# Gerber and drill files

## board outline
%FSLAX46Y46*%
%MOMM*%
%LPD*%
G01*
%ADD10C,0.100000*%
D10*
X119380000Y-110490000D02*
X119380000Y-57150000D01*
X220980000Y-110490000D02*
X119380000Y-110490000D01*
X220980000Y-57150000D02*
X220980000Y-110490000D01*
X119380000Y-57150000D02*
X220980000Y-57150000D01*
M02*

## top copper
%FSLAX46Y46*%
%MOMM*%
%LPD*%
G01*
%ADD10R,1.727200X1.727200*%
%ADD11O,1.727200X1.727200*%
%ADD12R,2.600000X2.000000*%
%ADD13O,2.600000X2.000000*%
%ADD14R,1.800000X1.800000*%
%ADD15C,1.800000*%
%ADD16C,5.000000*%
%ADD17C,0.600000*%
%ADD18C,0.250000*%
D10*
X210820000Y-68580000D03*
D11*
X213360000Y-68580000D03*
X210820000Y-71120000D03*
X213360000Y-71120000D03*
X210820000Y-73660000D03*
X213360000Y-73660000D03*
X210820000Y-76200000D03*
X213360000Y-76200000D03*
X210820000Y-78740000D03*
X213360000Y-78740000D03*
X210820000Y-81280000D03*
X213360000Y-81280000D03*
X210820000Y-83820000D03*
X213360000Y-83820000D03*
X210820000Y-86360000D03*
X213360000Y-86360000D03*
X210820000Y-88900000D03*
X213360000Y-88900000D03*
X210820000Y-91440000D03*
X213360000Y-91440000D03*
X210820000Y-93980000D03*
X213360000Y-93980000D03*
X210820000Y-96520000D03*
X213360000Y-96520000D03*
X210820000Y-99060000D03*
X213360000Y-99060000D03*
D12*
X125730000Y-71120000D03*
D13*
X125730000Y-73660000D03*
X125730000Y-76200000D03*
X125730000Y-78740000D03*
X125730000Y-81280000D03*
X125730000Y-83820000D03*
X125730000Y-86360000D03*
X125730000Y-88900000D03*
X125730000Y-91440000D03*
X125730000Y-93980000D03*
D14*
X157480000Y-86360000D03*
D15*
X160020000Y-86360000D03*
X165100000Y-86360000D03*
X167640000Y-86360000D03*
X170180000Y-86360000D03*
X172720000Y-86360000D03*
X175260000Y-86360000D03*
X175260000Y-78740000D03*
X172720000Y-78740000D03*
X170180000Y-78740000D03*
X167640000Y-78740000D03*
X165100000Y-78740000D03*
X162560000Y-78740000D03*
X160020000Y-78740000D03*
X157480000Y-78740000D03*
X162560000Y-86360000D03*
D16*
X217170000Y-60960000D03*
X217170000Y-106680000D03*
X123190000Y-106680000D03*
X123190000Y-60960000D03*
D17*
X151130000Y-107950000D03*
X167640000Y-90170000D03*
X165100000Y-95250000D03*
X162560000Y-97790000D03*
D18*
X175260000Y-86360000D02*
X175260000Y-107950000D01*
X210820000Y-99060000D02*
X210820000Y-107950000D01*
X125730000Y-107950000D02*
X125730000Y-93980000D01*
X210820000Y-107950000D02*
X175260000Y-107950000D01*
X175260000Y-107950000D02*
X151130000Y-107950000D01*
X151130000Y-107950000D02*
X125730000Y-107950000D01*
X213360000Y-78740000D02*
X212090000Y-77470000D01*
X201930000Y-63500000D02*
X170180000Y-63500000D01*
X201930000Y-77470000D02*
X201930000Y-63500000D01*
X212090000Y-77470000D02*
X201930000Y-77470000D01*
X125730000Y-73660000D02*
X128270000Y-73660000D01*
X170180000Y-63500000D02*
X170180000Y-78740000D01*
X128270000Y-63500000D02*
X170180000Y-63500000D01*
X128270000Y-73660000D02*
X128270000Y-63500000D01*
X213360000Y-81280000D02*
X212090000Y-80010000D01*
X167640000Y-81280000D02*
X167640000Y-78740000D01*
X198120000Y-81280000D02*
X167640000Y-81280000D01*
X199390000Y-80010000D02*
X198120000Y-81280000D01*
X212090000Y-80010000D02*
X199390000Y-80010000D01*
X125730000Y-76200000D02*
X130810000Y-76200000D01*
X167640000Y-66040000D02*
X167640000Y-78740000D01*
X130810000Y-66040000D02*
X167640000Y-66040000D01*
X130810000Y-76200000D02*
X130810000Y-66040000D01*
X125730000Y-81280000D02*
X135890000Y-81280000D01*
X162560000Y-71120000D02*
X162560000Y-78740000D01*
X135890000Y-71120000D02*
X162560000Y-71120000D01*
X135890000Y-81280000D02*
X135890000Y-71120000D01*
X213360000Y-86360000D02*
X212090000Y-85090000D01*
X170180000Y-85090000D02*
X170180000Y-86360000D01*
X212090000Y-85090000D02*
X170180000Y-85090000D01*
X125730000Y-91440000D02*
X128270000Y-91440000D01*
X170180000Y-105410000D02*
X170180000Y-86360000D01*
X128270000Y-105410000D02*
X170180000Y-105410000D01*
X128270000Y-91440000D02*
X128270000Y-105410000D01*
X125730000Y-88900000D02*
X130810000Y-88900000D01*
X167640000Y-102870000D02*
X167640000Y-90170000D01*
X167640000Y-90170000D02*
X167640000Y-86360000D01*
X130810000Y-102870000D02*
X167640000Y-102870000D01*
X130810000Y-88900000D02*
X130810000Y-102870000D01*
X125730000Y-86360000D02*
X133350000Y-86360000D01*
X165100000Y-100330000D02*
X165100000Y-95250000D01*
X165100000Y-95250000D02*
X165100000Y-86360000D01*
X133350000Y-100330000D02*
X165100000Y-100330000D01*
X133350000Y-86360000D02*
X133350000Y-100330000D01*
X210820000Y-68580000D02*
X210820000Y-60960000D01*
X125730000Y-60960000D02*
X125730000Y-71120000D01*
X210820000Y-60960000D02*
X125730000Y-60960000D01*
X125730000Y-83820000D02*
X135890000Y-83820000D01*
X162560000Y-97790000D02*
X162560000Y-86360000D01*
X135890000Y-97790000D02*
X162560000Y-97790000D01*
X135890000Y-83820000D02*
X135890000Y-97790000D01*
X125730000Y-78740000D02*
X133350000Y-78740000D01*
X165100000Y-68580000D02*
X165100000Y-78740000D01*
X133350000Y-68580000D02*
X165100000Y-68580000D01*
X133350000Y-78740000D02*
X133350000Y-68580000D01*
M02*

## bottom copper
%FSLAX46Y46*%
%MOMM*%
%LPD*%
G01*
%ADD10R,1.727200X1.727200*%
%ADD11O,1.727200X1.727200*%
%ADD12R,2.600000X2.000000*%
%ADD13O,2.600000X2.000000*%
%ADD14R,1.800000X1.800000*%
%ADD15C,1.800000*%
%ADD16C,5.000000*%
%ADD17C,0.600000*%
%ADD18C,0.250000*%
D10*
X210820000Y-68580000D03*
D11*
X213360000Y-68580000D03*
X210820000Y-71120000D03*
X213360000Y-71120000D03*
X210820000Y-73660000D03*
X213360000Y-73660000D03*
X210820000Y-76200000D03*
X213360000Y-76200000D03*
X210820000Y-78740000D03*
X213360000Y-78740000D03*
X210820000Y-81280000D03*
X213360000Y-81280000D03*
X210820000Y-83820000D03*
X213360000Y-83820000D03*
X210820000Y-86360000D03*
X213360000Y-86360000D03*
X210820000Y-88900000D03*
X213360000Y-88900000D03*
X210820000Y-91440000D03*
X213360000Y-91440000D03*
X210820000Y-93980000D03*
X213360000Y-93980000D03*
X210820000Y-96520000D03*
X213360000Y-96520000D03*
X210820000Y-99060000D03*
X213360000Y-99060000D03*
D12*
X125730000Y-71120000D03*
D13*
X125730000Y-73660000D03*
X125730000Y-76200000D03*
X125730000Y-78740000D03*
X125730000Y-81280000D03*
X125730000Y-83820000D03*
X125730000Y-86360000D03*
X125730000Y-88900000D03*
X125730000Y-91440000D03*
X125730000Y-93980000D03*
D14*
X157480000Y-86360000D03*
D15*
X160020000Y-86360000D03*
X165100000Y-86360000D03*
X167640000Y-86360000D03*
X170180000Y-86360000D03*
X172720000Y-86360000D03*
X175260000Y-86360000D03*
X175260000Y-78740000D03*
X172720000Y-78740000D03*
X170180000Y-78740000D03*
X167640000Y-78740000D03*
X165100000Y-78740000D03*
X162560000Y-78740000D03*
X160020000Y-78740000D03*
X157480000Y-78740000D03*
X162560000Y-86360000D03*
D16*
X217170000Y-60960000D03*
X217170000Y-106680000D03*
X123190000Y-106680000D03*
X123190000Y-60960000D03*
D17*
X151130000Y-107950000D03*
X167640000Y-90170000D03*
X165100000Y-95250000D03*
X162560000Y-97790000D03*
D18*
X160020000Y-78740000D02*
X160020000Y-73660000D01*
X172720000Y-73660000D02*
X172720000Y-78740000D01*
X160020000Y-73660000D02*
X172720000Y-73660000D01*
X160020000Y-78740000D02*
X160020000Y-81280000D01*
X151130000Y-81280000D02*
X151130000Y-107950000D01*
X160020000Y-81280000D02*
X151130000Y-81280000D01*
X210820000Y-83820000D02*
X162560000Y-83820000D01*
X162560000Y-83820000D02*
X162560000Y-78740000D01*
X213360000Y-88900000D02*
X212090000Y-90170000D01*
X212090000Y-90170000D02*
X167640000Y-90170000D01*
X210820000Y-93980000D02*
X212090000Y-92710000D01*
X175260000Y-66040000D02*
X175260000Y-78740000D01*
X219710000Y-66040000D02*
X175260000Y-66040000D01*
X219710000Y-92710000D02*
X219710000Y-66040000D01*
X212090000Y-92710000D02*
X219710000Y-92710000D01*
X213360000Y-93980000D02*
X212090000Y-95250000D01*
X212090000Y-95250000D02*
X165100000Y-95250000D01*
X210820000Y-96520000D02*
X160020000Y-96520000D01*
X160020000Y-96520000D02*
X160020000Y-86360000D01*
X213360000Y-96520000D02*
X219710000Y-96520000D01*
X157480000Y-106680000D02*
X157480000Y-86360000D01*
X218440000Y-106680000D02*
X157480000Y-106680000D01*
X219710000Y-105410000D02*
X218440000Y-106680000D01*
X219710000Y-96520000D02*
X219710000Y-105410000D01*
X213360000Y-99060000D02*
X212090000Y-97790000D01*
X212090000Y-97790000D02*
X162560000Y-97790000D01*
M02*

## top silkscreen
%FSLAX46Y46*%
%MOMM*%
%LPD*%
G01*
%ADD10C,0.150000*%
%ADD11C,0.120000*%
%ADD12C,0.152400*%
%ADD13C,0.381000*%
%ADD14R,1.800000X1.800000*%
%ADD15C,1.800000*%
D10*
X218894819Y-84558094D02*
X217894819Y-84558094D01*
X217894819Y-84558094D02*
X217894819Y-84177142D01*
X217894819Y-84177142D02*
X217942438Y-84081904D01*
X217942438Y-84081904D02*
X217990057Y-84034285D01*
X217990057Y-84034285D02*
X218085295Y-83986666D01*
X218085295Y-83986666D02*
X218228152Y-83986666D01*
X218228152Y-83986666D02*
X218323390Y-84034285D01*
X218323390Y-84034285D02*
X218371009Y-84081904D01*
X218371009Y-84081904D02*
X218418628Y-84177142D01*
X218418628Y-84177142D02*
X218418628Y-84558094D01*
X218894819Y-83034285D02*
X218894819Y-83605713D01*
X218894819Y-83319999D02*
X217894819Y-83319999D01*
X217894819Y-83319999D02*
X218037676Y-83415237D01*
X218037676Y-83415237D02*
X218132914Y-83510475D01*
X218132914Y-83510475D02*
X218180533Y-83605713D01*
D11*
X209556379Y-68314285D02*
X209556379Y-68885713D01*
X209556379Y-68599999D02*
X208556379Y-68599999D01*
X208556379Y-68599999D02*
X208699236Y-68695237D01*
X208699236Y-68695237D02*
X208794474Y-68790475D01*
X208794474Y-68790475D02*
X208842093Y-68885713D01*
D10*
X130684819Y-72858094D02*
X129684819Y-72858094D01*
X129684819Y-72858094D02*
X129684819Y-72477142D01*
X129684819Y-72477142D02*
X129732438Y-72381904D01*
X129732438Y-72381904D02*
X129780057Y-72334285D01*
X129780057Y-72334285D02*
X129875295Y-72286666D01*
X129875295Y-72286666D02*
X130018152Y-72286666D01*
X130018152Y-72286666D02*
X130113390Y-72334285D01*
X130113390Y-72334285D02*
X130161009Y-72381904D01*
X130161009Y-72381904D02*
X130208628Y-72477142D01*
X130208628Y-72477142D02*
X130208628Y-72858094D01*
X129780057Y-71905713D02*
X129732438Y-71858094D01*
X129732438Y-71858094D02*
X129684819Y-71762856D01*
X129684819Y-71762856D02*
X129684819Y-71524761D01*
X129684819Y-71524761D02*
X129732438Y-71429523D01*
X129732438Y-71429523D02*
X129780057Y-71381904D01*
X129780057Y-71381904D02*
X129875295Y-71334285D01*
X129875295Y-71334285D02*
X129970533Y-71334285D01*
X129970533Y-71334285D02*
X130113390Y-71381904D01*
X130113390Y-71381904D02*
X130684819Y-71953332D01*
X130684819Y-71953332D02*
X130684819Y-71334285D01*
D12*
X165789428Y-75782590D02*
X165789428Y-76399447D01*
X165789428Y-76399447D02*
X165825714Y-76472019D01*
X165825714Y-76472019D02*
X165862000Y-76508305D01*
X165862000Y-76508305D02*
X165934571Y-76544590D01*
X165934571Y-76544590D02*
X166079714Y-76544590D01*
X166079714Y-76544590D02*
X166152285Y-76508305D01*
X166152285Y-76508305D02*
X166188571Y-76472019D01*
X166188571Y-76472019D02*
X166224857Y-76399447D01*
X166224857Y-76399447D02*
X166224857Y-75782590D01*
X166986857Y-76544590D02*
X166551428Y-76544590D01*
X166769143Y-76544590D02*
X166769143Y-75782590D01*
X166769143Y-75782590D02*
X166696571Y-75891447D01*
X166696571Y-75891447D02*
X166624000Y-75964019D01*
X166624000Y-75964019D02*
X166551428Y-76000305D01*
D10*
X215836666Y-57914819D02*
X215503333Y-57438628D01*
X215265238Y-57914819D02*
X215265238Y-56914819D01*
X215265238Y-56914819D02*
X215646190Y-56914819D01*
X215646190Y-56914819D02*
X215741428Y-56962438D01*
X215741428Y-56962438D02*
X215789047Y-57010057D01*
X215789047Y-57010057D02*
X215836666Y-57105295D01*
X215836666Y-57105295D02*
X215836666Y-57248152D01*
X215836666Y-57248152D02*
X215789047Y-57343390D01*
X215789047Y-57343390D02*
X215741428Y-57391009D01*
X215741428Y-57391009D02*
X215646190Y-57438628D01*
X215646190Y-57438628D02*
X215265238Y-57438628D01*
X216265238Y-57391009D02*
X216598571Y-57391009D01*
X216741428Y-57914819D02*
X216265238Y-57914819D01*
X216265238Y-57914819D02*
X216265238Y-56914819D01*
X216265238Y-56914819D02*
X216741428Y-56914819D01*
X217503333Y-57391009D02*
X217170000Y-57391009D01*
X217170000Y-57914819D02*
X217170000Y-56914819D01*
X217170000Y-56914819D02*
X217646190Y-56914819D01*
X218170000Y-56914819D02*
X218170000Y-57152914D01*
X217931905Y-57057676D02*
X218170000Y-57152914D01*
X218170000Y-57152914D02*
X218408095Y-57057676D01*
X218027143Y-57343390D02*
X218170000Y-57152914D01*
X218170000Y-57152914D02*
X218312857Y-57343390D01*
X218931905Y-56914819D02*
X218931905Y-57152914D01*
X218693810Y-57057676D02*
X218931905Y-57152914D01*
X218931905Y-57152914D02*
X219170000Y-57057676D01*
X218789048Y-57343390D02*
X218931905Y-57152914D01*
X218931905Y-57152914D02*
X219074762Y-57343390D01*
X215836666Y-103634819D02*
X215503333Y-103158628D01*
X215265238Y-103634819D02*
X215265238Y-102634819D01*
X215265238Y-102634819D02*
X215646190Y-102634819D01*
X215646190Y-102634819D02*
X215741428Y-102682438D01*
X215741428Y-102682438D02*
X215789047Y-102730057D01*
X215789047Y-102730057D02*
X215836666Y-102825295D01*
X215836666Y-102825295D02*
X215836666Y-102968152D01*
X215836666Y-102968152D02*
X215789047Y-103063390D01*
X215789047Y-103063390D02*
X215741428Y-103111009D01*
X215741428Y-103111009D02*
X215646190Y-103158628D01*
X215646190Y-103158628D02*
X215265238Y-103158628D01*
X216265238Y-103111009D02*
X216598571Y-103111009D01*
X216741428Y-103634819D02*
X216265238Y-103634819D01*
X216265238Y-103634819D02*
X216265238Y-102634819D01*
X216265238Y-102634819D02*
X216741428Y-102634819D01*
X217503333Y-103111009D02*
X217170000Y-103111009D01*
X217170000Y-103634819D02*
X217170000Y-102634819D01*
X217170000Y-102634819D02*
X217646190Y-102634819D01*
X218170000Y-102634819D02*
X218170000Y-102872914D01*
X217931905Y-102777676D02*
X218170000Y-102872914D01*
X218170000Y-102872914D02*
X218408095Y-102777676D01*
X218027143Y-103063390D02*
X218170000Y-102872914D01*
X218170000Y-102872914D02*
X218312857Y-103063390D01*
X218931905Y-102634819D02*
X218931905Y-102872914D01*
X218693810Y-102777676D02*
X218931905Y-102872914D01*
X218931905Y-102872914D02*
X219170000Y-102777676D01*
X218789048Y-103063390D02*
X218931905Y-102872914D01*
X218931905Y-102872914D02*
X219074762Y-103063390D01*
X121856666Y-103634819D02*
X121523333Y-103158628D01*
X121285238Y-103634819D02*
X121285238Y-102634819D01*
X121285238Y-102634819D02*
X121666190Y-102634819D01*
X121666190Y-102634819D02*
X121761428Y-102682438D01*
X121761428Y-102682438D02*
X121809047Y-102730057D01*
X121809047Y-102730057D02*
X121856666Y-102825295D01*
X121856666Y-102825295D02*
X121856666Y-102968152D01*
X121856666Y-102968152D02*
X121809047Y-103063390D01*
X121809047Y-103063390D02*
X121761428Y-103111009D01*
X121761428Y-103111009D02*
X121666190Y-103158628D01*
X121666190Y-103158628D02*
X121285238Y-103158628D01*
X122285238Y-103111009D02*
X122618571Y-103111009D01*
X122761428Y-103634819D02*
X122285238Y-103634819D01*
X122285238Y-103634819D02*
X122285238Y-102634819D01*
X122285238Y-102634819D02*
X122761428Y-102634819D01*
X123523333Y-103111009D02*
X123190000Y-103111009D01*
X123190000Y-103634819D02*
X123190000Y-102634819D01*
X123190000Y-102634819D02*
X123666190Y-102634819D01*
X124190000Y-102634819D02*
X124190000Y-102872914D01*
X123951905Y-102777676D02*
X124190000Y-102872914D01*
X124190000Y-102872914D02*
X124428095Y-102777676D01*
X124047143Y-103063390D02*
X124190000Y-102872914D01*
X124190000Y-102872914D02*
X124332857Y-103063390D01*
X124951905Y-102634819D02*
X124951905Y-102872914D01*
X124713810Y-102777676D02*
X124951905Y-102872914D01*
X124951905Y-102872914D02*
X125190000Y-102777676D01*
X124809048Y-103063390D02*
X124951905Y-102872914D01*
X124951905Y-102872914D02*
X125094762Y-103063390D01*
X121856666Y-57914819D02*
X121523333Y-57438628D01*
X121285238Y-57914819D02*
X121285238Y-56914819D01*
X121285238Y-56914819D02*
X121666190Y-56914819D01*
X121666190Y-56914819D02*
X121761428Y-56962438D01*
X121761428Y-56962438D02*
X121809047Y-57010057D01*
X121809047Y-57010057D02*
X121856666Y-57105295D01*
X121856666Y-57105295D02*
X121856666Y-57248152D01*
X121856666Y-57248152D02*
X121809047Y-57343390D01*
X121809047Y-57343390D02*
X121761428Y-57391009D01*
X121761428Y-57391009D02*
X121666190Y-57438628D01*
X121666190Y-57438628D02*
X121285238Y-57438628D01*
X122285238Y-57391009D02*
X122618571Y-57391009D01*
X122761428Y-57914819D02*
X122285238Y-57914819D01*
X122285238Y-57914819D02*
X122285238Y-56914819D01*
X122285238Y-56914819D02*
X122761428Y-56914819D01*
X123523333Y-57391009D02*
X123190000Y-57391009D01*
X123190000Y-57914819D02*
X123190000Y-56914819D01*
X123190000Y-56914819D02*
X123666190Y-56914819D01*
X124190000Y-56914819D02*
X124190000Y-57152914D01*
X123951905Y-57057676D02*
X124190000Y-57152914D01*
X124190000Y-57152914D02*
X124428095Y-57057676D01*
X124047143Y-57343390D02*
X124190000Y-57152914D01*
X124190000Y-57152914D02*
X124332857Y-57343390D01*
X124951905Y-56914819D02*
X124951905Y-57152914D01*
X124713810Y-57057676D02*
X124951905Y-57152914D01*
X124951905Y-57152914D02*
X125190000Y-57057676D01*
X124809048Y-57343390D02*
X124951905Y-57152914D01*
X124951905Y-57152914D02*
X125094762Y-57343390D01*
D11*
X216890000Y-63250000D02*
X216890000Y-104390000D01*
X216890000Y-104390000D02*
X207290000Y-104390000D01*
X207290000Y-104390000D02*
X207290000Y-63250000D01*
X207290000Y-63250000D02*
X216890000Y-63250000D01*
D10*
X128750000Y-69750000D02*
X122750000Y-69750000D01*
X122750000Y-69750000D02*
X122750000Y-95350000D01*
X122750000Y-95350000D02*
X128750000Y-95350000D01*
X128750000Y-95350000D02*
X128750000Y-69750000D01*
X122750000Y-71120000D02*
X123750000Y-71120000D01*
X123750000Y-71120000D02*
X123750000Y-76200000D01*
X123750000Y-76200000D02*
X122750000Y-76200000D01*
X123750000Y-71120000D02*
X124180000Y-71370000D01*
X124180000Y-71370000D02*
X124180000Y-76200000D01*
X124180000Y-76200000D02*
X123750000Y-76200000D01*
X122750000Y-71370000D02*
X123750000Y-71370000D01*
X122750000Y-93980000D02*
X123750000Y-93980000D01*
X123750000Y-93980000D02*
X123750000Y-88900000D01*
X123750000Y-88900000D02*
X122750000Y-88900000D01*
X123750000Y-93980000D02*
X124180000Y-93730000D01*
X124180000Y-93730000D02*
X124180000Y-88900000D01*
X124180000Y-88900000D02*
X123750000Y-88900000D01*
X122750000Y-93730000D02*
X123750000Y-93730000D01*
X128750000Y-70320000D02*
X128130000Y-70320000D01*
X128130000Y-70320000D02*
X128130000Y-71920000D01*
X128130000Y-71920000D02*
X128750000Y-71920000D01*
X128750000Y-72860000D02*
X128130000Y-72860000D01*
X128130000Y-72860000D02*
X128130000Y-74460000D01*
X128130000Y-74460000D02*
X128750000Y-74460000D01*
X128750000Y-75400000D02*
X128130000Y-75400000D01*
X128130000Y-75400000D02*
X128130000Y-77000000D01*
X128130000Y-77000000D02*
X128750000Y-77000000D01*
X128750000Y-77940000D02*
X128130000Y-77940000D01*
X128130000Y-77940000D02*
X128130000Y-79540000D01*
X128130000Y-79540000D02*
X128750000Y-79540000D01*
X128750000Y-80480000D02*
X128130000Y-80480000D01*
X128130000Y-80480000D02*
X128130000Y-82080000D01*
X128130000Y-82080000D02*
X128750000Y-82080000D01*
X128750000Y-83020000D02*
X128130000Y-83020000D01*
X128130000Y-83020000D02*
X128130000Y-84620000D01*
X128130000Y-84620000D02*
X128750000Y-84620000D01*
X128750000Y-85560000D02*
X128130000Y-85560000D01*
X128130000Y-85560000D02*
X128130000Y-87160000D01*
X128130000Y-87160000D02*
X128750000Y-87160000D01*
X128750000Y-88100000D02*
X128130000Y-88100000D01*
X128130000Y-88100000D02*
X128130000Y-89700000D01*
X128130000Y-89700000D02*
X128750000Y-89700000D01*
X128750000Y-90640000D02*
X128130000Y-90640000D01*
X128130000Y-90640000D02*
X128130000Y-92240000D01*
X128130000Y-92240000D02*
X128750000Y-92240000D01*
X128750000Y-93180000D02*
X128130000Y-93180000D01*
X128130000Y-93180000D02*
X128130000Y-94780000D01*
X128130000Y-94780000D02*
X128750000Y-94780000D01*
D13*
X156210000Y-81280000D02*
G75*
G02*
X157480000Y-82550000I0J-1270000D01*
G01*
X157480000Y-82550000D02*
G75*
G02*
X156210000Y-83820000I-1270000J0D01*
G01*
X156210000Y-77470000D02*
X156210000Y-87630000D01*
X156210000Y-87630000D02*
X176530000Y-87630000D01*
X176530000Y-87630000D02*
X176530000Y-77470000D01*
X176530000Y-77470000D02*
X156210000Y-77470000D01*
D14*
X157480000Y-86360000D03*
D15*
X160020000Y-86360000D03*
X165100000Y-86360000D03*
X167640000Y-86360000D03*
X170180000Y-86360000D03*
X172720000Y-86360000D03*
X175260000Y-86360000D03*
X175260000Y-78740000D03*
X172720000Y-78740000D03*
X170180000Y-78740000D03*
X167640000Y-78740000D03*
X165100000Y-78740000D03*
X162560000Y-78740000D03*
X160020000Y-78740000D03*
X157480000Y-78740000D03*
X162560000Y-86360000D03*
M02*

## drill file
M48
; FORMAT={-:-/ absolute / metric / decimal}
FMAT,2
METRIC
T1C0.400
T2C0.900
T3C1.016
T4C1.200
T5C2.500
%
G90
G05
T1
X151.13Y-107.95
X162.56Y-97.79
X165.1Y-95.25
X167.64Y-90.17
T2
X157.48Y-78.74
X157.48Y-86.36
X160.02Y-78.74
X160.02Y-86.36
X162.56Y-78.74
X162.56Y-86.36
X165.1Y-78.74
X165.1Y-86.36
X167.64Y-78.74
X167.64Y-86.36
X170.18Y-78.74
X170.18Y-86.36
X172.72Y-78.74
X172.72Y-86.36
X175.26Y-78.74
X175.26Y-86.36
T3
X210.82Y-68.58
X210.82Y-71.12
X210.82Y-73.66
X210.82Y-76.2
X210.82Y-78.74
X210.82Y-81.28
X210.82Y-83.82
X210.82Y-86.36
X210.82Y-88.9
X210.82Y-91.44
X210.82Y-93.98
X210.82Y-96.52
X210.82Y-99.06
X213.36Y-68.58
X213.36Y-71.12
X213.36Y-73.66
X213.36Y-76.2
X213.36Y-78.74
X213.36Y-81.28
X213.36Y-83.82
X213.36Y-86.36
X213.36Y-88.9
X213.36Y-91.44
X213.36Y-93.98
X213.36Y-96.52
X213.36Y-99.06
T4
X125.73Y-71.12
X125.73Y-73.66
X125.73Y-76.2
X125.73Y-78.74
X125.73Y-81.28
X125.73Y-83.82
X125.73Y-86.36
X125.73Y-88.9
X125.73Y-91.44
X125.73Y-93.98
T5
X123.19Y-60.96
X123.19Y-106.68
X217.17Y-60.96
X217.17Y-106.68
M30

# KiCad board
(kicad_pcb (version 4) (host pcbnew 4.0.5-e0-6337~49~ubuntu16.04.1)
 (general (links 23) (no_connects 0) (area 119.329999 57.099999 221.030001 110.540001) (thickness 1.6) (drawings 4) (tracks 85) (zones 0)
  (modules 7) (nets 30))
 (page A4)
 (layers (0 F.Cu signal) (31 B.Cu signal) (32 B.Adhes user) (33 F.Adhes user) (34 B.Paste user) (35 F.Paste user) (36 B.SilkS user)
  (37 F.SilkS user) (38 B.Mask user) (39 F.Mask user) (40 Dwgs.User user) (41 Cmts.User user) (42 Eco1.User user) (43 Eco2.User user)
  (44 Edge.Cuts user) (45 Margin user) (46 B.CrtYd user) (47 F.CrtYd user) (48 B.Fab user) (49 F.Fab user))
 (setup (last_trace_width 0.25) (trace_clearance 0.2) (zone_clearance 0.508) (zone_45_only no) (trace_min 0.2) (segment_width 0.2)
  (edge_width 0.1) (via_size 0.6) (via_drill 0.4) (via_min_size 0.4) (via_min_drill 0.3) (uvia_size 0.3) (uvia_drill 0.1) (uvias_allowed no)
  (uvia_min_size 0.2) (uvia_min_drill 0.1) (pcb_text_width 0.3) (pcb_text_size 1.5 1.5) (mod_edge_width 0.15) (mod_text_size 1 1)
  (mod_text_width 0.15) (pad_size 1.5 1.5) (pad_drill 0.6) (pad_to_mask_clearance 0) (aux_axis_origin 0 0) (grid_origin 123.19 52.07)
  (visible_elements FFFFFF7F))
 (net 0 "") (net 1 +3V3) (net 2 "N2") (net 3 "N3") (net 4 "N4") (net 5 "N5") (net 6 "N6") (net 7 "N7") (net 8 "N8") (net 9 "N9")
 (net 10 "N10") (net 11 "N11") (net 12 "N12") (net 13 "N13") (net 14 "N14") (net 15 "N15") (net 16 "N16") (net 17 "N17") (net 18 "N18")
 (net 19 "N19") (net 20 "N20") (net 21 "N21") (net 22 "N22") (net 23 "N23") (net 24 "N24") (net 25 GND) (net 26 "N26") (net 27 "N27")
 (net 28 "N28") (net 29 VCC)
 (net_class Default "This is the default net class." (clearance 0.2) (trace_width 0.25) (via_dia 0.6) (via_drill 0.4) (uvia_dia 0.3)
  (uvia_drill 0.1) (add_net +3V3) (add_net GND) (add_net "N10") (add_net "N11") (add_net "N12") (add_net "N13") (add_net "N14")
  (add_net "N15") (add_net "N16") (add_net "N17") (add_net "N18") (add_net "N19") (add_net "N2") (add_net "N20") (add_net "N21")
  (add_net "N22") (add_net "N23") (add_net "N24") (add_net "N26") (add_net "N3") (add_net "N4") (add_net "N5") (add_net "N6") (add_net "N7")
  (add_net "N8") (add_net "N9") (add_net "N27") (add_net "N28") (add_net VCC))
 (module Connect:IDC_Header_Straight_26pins (layer F.Cu) (at 210.82 68.58 270)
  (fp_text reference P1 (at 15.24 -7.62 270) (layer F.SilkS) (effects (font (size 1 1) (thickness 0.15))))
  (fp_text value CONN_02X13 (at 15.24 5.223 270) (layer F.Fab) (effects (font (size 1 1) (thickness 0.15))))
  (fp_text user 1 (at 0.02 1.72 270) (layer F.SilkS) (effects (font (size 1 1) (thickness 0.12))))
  (fp_line (start -5.33 -6.07) (end 35.81 -6.07) (layer F.SilkS) (width 0.12))
  (fp_line (start 35.81 -6.07) (end 35.81 3.53) (layer F.SilkS) (width 0.12))
  (fp_line (start 35.81 3.53) (end -5.33 3.53) (layer F.SilkS) (width 0.12))
  (fp_line (start -5.33 3.53) (end -5.33 -6.07) (layer F.SilkS) (width 0.12))
  (pad 1 thru_hole rect (at 0 0 270) (size 1.7272 1.7272) (drill 1.016) (layers *.Cu *.Mask) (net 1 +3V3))
  (pad 2 thru_hole oval (at 0 -2.54 270) (size 1.7272 1.7272) (drill 1.016) (layers *.Cu *.Mask) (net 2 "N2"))
  (pad 3 thru_hole oval (at 2.54 0 270) (size 1.7272 1.7272) (drill 1.016) (layers *.Cu *.Mask) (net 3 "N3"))
  (pad 4 thru_hole oval (at 2.54 -2.54 270) (size 1.7272 1.7272) (drill 1.016) (layers *.Cu *.Mask) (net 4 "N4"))
  (pad 5 thru_hole oval (at 5.08 0 270) (size 1.7272 1.7272) (drill 1.016) (layers *.Cu *.Mask) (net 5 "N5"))
  (pad 6 thru_hole oval (at 5.08 -2.54 270) (size 1.7272 1.7272) (drill 1.016) (layers *.Cu *.Mask) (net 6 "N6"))
  (pad 7 thru_hole oval (at 7.62 0 270) (size 1.7272 1.7272) (drill 1.016) (layers *.Cu *.Mask) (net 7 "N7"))
  (pad 8 thru_hole oval (at 7.62 -2.54 270) (size 1.7272 1.7272) (drill 1.016) (layers *.Cu *.Mask) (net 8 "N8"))
  (pad 9 thru_hole oval (at 10.16 0 270) (size 1.7272 1.7272) (drill 1.016) (layers *.Cu *.Mask) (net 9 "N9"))
  (pad 10 thru_hole oval (at 10.16 -2.54 270) (size 1.7272 1.7272) (drill 1.016) (layers *.Cu *.Mask) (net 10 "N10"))
  (pad 11 thru_hole oval (at 12.7 0 270) (size 1.7272 1.7272) (drill 1.016) (layers *.Cu *.Mask) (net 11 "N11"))
  (pad 12 thru_hole oval (at 12.7 -2.54 270) (size 1.7272 1.7272) (drill 1.016) (layers *.Cu *.Mask) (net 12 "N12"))
  (pad 13 thru_hole oval (at 15.24 0 270) (size 1.7272 1.7272) (drill 1.016) (layers *.Cu *.Mask) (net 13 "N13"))
  (pad 14 thru_hole oval (at 15.24 -2.54 270) (size 1.7272 1.7272) (drill 1.016) (layers *.Cu *.Mask) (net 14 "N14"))
  (pad 15 thru_hole oval (at 17.78 0 270) (size 1.7272 1.7272) (drill 1.016) (layers *.Cu *.Mask) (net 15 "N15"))
  (pad 16 thru_hole oval (at 17.78 -2.54 270) (size 1.7272 1.7272) (drill 1.016) (layers *.Cu *.Mask) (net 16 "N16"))
  (pad 17 thru_hole oval (at 20.32 0 270) (size 1.7272 1.7272) (drill 1.016) (layers *.Cu *.Mask) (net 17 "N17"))
  (pad 18 thru_hole oval (at 20.32 -2.54 270) (size 1.7272 1.7272) (drill 1.016) (layers *.Cu *.Mask) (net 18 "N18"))
  (pad 19 thru_hole oval (at 22.86 0 270) (size 1.7272 1.7272) (drill 1.016) (layers *.Cu *.Mask) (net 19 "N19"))
  (pad 20 thru_hole oval (at 22.86 -2.54 270) (size 1.7272 1.7272) (drill 1.016) (layers *.Cu *.Mask) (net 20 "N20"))
  (pad 21 thru_hole oval (at 25.4 0 270) (size 1.7272 1.7272) (drill 1.016) (layers *.Cu *.Mask) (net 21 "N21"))
  (pad 22 thru_hole oval (at 25.4 -2.54 270) (size 1.7272 1.7272) (drill 1.016) (layers *.Cu *.Mask) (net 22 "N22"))
  (pad 23 thru_hole oval (at 27.94 0 270) (size 1.7272 1.7272) (drill 1.016) (layers *.Cu *.Mask) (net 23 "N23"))
  (pad 24 thru_hole oval (at 27.94 -2.54 270) (size 1.7272 1.7272) (drill 1.016) (layers *.Cu *.Mask) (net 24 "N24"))
  (pad 25 thru_hole oval (at 30.48 0 270) (size 1.7272 1.7272) (drill 1.016) (layers *.Cu *.Mask) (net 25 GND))
  (pad 26 thru_hole oval (at 30.48 -2.54 270) (size 1.7272 1.7272) (drill 1.016) (layers *.Cu *.Mask) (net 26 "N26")))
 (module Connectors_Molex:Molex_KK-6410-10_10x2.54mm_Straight (layer F.Cu) (at 125.73 71.12 270)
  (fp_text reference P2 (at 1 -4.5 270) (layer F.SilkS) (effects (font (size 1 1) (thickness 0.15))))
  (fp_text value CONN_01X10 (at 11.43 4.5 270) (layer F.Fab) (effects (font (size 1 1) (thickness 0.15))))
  (fp_line (start -1.37 -3.02) (end -1.37 2.98) (layer F.SilkS) (width 0.15))
  (fp_line (start -1.37 2.98) (end 24.23 2.98) (layer F.SilkS) (width 0.15))
  (fp_line (start 24.23 2.98) (end 24.23 -3.02) (layer F.SilkS) (width 0.15))
  (fp_line (start 24.23 -3.02) (end -1.37 -3.02) (layer F.SilkS) (width 0.15))
  (fp_line (start 0 2.98) (end 0 1.98) (layer F.SilkS) (width 0.15))
  (fp_line (start 0 1.98) (end 5.08 1.98) (layer F.SilkS) (width 0.15))
  (fp_line (start 5.08 1.98) (end 5.08 2.98) (layer F.SilkS) (width 0.15))
  (fp_line (start 0 1.98) (end 0.25 1.55) (layer F.SilkS) (width 0.15))
  (fp_line (start 0.25 1.55) (end 5.08 1.55) (layer F.SilkS) (width 0.15))
  (fp_line (start 5.08 1.55) (end 5.08 1.98) (layer F.SilkS) (width 0.15))
  (fp_line (start 0.25 2.98) (end 0.25 1.98) (layer F.SilkS) (width 0.15))
  (fp_line (start 22.86 2.98) (end 22.86 1.98) (layer F.SilkS) (width 0.15))
  (fp_line (start 22.86 1.98) (end 17.78 1.98) (layer F.SilkS) (width 0.15))
  (fp_line (start 17.78 1.98) (end 17.78 2.98) (layer F.SilkS) (width 0.15))
  (fp_line (start 22.86 1.98) (end 22.61 1.55) (layer F.SilkS) (width 0.15))
  (fp_line (start 22.61 1.55) (end 17.78 1.55) (layer F.SilkS) (width 0.15))
  (fp_line (start 17.78 1.55) (end 17.78 1.98) (layer F.SilkS) (width 0.15))
  (fp_line (start 22.61 2.98) (end 22.61 1.98) (layer F.SilkS) (width 0.15))
  (fp_line (start -0.8 -3.02) (end -0.8 -2.4) (layer F.SilkS) (width 0.15))
  (fp_line (start -0.8 -2.4) (end 0.8 -2.4) (layer F.SilkS) (width 0.15))
  (fp_line (start 0.8 -2.4) (end 0.8 -3.02) (layer F.SilkS) (width 0.15))
  (fp_line (start 1.74 -3.02) (end 1.74 -2.4) (layer F.SilkS) (width 0.15))
  (fp_line (start 1.74 -2.4) (end 3.34 -2.4) (layer F.SilkS) (width 0.15))
  (fp_line (start 3.34 -2.4) (end 3.34 -3.02) (layer F.SilkS) (width 0.15))
  (fp_line (start 4.28 -3.02) (end 4.28 -2.4) (layer F.SilkS) (width 0.15))
  (fp_line (start 4.28 -2.4) (end 5.88 -2.4) (layer F.SilkS) (width 0.15))
  (fp_line (start 5.88 -2.4) (end 5.88 -3.02) (layer F.SilkS) (width 0.15))
  (fp_line (start 6.82 -3.02) (end 6.82 -2.4) (layer F.SilkS) (width 0.15))
  (fp_line (start 6.82 -2.4) (end 8.42 -2.4) (layer F.SilkS) (width 0.15))
  (fp_line (start 8.42 -2.4) (end 8.42 -3.02) (layer F.SilkS) (width 0.15))
  (fp_line (start 9.36 -3.02) (end 9.36 -2.4) (layer F.SilkS) (width 0.15))
  (fp_line (start 9.36 -2.4) (end 10.96 -2.4) (layer F.SilkS) (width 0.15))
  (fp_line (start 10.96 -2.4) (end 10.96 -3.02) (layer F.SilkS) (width 0.15))
  (fp_line (start 11.9 -3.02) (end 11.9 -2.4) (layer F.SilkS) (width 0.15))
  (fp_line (start 11.9 -2.4) (end 13.5 -2.4) (layer F.SilkS) (width 0.15))
  (fp_line (start 13.5 -2.4) (end 13.5 -3.02) (layer F.SilkS) (width 0.15))
  (fp_line (start 14.44 -3.02) (end 14.44 -2.4) (layer F.SilkS) (width 0.15))
  (fp_line (start 14.44 -2.4) (end 16.04 -2.4) (layer F.SilkS) (width 0.15))
  (fp_line (start 16.04 -2.4) (end 16.04 -3.02) (layer F.SilkS) (width 0.15))
  (fp_line (start 16.98 -3.02) (end 16.98 -2.4) (layer F.SilkS) (width 0.15))
  (fp_line (start 16.98 -2.4) (end 18.58 -2.4) (layer F.SilkS) (width 0.15))
  (fp_line (start 18.58 -2.4) (end 18.58 -3.02) (layer F.SilkS) (width 0.15))
  (fp_line (start 19.52 -3.02) (end 19.52 -2.4) (layer F.SilkS) (width 0.15))
  (fp_line (start 19.52 -2.4) (end 21.12 -2.4) (layer F.SilkS) (width 0.15))
  (fp_line (start 21.12 -2.4) (end 21.12 -3.02) (layer F.SilkS) (width 0.15))
  (fp_line (start 22.06 -3.02) (end 22.06 -2.4) (layer F.SilkS) (width 0.15))
  (fp_line (start 22.06 -2.4) (end 23.66 -2.4) (layer F.SilkS) (width 0.15))
  (fp_line (start 23.66 -2.4) (end 23.66 -3.02) (layer F.SilkS) (width 0.15))
  (pad 1 thru_hole rect (at 0 0 270) (size 2 2.6) (drill 1.2) (layers *.Cu *.Mask) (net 1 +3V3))
  (pad 2 thru_hole oval (at 2.54 0 270) (size 2 2.6) (drill 1.2) (layers *.Cu *.Mask) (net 10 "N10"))
  (pad 3 thru_hole oval (at 5.08 0 270) (size 2 2.6) (drill 1.2) (layers *.Cu *.Mask) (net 12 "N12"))
  (pad 4 thru_hole oval (at 7.62 0 270) (size 2 2.6) (drill 1.2) (layers *.Cu *.Mask) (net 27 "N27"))
  (pad 5 thru_hole oval (at 10.16 0 270) (size 2 2.6) (drill 1.2) (layers *.Cu *.Mask) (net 13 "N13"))
  (pad 6 thru_hole oval (at 12.7 0 270) (size 2 2.6) (drill 1.2) (layers *.Cu *.Mask) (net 26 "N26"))
  (pad 7 thru_hole oval (at 15.24 0 270) (size 2 2.6) (drill 1.2) (layers *.Cu *.Mask) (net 22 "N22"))
  (pad 8 thru_hole oval (at 17.78 0 270) (size 2 2.6) (drill 1.2) (layers *.Cu *.Mask) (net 18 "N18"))
  (pad 9 thru_hole oval (at 20.32 0 270) (size 2 2.6) (drill 1.2) (layers *.Cu *.Mask) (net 16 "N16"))
  (pad 10 thru_hole oval (at 22.86 0 270) (size 2 2.6) (drill 1.2) (layers *.Cu *.Mask) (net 25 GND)))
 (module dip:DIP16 (layer F.Cu) (at 166.37 82.55)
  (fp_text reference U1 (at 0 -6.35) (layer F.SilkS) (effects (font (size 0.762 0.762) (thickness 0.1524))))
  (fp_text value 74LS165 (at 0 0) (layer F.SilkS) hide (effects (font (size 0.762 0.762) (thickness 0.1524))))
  (fp_arc (start -10.16 0) (end -10.16 -1.27) (angle 90) (layer F.SilkS) (width 0.381))
  (fp_arc (start -10.16 0) (end -8.89 0) (angle 90) (layer F.SilkS) (width 0.381))
  (fp_line (start -10.16 -5.08) (end -10.16 5.08) (layer F.SilkS) (width 0.381))
  (fp_line (start -10.16 5.08) (end 10.16 5.08) (layer F.SilkS) (width 0.381))
  (fp_line (start 10.16 5.08) (end 10.16 -5.08) (layer F.SilkS) (width 0.381))
  (fp_line (start 10.16 -5.08) (end -10.16 -5.08) (layer F.SilkS) (width 0.381))
  (pad 1 thru_hole rect (at -8.89 3.81) (size 1.8 1.8) (drill 0.9) (layers *.Cu *.Mask F.SilkS) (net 24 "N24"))
  (pad 2 thru_hole circle (at -6.35 3.81) (size 1.8 1.8) (drill 0.9) (layers *.Cu *.Mask F.SilkS) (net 23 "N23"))
  (pad 4 thru_hole circle (at -1.27 3.81) (size 1.8 1.8) (drill 0.9) (layers *.Cu *.Mask F.SilkS) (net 22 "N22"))
  (pad 5 thru_hole circle (at 1.27 3.81) (size 1.8 1.8) (drill 0.9) (layers *.Cu *.Mask F.SilkS) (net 18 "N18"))
  (pad 6 thru_hole circle (at 3.81 3.81) (size 1.8 1.8) (drill 0.9) (layers *.Cu *.Mask F.SilkS) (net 16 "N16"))
  (pad 7 thru_hole circle (at 6.35 3.81) (size 1.8 1.8) (drill 0.9) (layers *.Cu *.Mask F.SilkS) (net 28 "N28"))
  (pad 8 thru_hole circle (at 8.89 3.81) (size 1.8 1.8) (drill 0.9) (layers *.Cu *.Mask F.SilkS) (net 25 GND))
  (pad 9 thru_hole circle (at 8.89 -3.81) (size 1.8 1.8) (drill 0.9) (layers *.Cu *.Mask F.SilkS) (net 21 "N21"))
  (pad 10 thru_hole circle (at 6.35 -3.81) (size 1.8 1.8) (drill 0.9) (layers *.Cu *.Mask F.SilkS) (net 25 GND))
  (pad 11 thru_hole circle (at 3.81 -3.81) (size 1.8 1.8) (drill 0.9) (layers *.Cu *.Mask F.SilkS) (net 10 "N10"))
  (pad 12 thru_hole circle (at 1.27 -3.81) (size 1.8 1.8) (drill 0.9) (layers *.Cu *.Mask F.SilkS) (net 12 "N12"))
  (pad 13 thru_hole circle (at -1.27 -3.81) (size 1.8 1.8) (drill 0.9) (layers *.Cu *.Mask F.SilkS) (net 27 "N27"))
  (pad 14 thru_hole circle (at -3.81 -3.81) (size 1.8 1.8) (drill 0.9) (layers *.Cu *.Mask F.SilkS) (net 13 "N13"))
  (pad 15 thru_hole circle (at -6.35 -3.81) (size 1.8 1.8) (drill 0.9) (layers *.Cu *.Mask F.SilkS) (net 25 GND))
  (pad 16 thru_hole circle (at -8.89 -3.81) (size 1.8 1.8) (drill 0.9) (layers *.Cu *.Mask F.SilkS) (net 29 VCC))
  (pad 3 thru_hole circle (at -3.81 3.81) (size 1.8 1.8) (drill 0.9) (layers *.Cu *.Mask F.SilkS) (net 26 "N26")))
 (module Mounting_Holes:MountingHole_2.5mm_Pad (layer F.Cu) (at 217.17 60.96)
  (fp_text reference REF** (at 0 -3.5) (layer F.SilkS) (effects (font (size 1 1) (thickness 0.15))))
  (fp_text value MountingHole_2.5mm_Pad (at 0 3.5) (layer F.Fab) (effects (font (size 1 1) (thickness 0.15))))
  (pad 1 thru_hole circle (at 0 0) (size 5 5) (drill 2.5) (layers *.Cu *.Mask)))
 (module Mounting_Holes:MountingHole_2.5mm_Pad (layer F.Cu) (at 217.17 106.68)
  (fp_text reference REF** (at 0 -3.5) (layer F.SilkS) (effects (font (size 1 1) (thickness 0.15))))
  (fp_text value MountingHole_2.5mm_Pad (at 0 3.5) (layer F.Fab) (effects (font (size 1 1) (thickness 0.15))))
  (pad 1 thru_hole circle (at 0 0) (size 5 5) (drill 2.5) (layers *.Cu *.Mask)))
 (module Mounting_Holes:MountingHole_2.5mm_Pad (layer F.Cu) (at 123.19 106.68)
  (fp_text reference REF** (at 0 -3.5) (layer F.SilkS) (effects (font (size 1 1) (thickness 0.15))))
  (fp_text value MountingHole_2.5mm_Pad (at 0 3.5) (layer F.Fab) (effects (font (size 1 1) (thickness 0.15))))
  (pad 1 thru_hole circle (at 0 0) (size 5 5) (drill 2.5) (layers *.Cu *.Mask)))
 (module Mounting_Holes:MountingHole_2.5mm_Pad (layer F.Cu) (at 123.19 60.96)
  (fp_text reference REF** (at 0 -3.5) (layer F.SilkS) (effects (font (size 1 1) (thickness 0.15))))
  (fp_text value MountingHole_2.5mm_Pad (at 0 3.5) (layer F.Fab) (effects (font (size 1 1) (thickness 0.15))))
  (pad 1 thru_hole circle (at 0 0) (size 5 5) (drill 2.5) (layers *.Cu *.Mask)))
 (gr_line (start 119.38 110.49) (end 119.38 57.15) (angle 90) (layer Edge.Cuts) (width 0.1))
 (gr_line (start 220.98 110.49) (end 119.38 110.49) (angle 90) (layer Edge.Cuts) (width 0.1))
 (gr_line (start 220.98 57.15) (end 220.98 110.49) (angle 90) (layer Edge.Cuts) (width 0.1))
 (gr_line (start 119.38 57.15) (end 220.98 57.15) (angle 90) (layer Edge.Cuts) (width 0.1))
 (segment (start 160.02 78.74) (end 160.02 73.66) (width 0.25) (layer B.Cu) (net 25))
 (segment (start 172.72 73.66) (end 172.72 78.74) (width 0.25) (layer B.Cu) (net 25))
 (segment (start 160.02 73.66) (end 172.72 73.66) (width 0.25) (layer B.Cu) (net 25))
 (segment (start 160.02 78.74) (end 160.02 81.28) (width 0.25) (layer B.Cu) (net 25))
 (via (at 151.13 107.95) (size 0.6) (drill 0.4) (layers F.Cu B.Cu) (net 25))
 (segment (start 151.13 81.28) (end 151.13 107.95) (width 0.25) (layer B.Cu) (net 25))
 (segment (start 160.02 81.28) (end 151.13 81.28) (width 0.25) (layer B.Cu) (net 25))
 (segment (start 175.26 86.36) (end 175.26 107.95) (width 0.25) (layer F.Cu) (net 25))
 (segment (start 210.82 99.06) (end 210.82 107.95) (width 0.25) (layer F.Cu) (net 25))
 (segment (start 125.73 107.95) (end 125.73 93.98) (width 0.25) (layer F.Cu) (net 25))
 (segment (start 210.82 107.95) (end 175.26 107.95) (width 0.25) (layer F.Cu) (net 25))
 (segment (start 175.26 107.95) (end 151.13 107.95) (width 0.25) (layer F.Cu) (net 25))
 (segment (start 151.13 107.95) (end 125.73 107.95) (width 0.25) (layer F.Cu) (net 25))
 (segment (start 213.36 78.74) (end 212.09 77.47) (width 0.25) (layer F.Cu) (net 10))
 (segment (start 201.93 63.5) (end 170.18 63.5) (width 0.25) (layer F.Cu) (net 10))
 (segment (start 201.93 77.47) (end 201.93 63.5) (width 0.25) (layer F.Cu) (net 10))
 (segment (start 212.09 77.47) (end 201.93 77.47) (width 0.25) (layer F.Cu) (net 10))
 (segment (start 125.73 73.66) (end 128.27 73.66) (width 0.25) (layer F.Cu) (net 10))
 (segment (start 170.18 63.5) (end 170.18 78.74) (width 0.25) (layer F.Cu) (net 10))
 (segment (start 128.27 63.5) (end 170.18 63.5) (width 0.25) (layer F.Cu) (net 10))
 (segment (start 128.27 73.66) (end 128.27 63.5) (width 0.25) (layer F.Cu) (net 10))
 (segment (start 213.36 81.28) (end 212.09 80.01) (width 0.25) (layer F.Cu) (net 12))
 (segment (start 167.64 81.28) (end 167.64 78.74) (width 0.25) (layer F.Cu) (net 12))
 (segment (start 198.12 81.28) (end 167.64 81.28) (width 0.25) (layer F.Cu) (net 12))
 (segment (start 199.39 80.01) (end 198.12 81.28) (width 0.25) (layer F.Cu) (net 12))
 (segment (start 212.09 80.01) (end 199.39 80.01) (width 0.25) (layer F.Cu) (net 12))
 (segment (start 125.73 76.2) (end 130.81 76.2) (width 0.25) (layer F.Cu) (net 12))
 (segment (start 167.64 66.04) (end 167.64 78.74) (width 0.25) (layer F.Cu) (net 12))
 (segment (start 130.81 66.04) (end 167.64 66.04) (width 0.25) (layer F.Cu) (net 12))
 (segment (start 130.81 76.2) (end 130.81 66.04) (width 0.25) (layer F.Cu) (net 12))
 (segment (start 210.82 83.82) (end 162.56 83.82) (width 0.25) (layer B.Cu) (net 13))
 (segment (start 162.56 83.82) (end 162.56 78.74) (width 0.25) (layer B.Cu) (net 13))
 (segment (start 125.73 81.28) (end 135.89 81.28) (width 0.25) (layer F.Cu) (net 13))
 (segment (start 162.56 71.12) (end 162.56 78.74) (width 0.25) (layer F.Cu) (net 13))
 (segment (start 135.89 71.12) (end 162.56 71.12) (width 0.25) (layer F.Cu) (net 13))
 (segment (start 135.89 81.28) (end 135.89 71.12) (width 0.25) (layer F.Cu) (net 13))
 (segment (start 213.36 86.36) (end 212.09 85.09) (width 0.25) (layer F.Cu) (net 16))
 (segment (start 170.18 85.09) (end 170.18 86.36) (width 0.25) (layer F.Cu) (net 16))
 (segment (start 212.09 85.09) (end 170.18 85.09) (width 0.25) (layer F.Cu) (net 16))
 (segment (start 125.73 91.44) (end 128.27 91.44) (width 0.25) (layer F.Cu) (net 16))
 (segment (start 170.18 105.41) (end 170.18 86.36) (width 0.25) (layer F.Cu) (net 16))
 (segment (start 128.27 105.41) (end 170.18 105.41) (width 0.25) (layer F.Cu) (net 16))
 (segment (start 128.27 91.44) (end 128.27 105.41) (width 0.25) (layer F.Cu) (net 16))
 (via (at 167.64 90.17) (size 0.6) (drill 0.4) (layers F.Cu B.Cu) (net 18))
 (segment (start 213.36 88.9) (end 212.09 90.17) (width 0.25) (layer B.Cu) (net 18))
 (segment (start 212.09 90.17) (end 167.64 90.17) (width 0.25) (layer B.Cu) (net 18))
 (segment (start 125.73 88.9) (end 130.81 88.9) (width 0.25) (layer F.Cu) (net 18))
 (segment (start 167.64 102.87) (end 167.64 90.17) (width 0.25) (layer F.Cu) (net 18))
 (segment (start 167.64 90.17) (end 167.64 86.36) (width 0.25) (layer F.Cu) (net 18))
 (segment (start 130.81 102.87) (end 167.64 102.87) (width 0.25) (layer F.Cu) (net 18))
 (segment (start 130.81 88.9) (end 130.81 102.87) (width 0.25) (layer F.Cu) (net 18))
 (segment (start 210.82 93.98) (end 212.09 92.71) (width 0.25) (layer B.Cu) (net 21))
 (segment (start 175.26 66.04) (end 175.26 78.74) (width 0.25) (layer B.Cu) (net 21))
 (segment (start 219.71 66.04) (end 175.26 66.04) (width 0.25) (layer B.Cu) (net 21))
 (segment (start 219.71 92.71) (end 219.71 66.04) (width 0.25) (layer B.Cu) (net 21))
 (segment (start 212.09 92.71) (end 219.71 92.71) (width 0.25) (layer B.Cu) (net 21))
 (via (at 165.1 95.25) (size 0.6) (drill 0.4) (layers F.Cu B.Cu) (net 22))
 (segment (start 213.36 93.98) (end 212.09 95.25) (width 0.25) (layer B.Cu) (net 22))
 (segment (start 212.09 95.25) (end 165.1 95.25) (width 0.25) (layer B.Cu) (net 22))
 (segment (start 125.73 86.36) (end 133.35 86.36) (width 0.25) (layer F.Cu) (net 22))
 (segment (start 165.1 100.33) (end 165.1 95.25) (width 0.25) (layer F.Cu) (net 22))
 (segment (start 165.1 95.25) (end 165.1 86.36) (width 0.25) (layer F.Cu) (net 22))
 (segment (start 133.35 100.33) (end 165.1 100.33) (width 0.25) (layer F.Cu) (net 22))
 (segment (start 133.35 86.36) (end 133.35 100.33) (width 0.25) (layer F.Cu) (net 22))
 (segment (start 210.82 96.52) (end 160.02 96.52) (width 0.25) (layer B.Cu) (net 23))
 (segment (start 160.02 96.52) (end 160.02 86.36) (width 0.25) (layer B.Cu) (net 23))
 (segment (start 213.36 96.52) (end 219.71 96.52) (width 0.25) (layer B.Cu) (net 24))
 (segment (start 157.48 106.68) (end 157.48 86.36) (width 0.25) (layer B.Cu) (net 24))
 (segment (start 218.44 106.68) (end 157.48 106.68) (width 0.25) (layer B.Cu) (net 24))
 (segment (start 219.71 105.41) (end 218.44 106.68) (width 0.25) (layer B.Cu) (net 24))
 (segment (start 219.71 96.52) (end 219.71 105.41) (width 0.25) (layer B.Cu) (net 24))
 (segment (start 210.82 68.58) (end 210.82 60.96) (width 0.25) (layer F.Cu) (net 1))
 (segment (start 125.73 60.96) (end 125.73 71.12) (width 0.25) (layer F.Cu) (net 1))
 (segment (start 210.82 60.96) (end 125.73 60.96) (width 0.25) (layer F.Cu) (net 1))
 (via (at 162.56 97.79) (size 0.6) (drill 0.4) (layers F.Cu B.Cu) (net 26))
 (segment (start 213.36 99.06) (end 212.09 97.79) (width 0.25) (layer B.Cu) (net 26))
 (segment (start 212.09 97.79) (end 162.56 97.79) (width 0.25) (layer B.Cu) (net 26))
 (segment (start 125.73 83.82) (end 135.89 83.82) (width 0.25) (layer F.Cu) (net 26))
 (segment (start 162.56 97.79) (end 162.56 86.36) (width 0.25) (layer F.Cu) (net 26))
 (segment (start 135.89 97.79) (end 162.56 97.79) (width 0.25) (layer F.Cu) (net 26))
 (segment (start 135.89 83.82) (end 135.89 97.79) (width 0.25) (layer F.Cu) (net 26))
 (segment (start 125.73 78.74) (end 133.35 78.74) (width 0.25) (layer F.Cu) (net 27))
 (segment (start 165.1 68.58) (end 165.1 78.74) (width 0.25) (layer F.Cu) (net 27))
 (segment (start 133.35 68.58) (end 165.1 68.58) (width 0.25) (layer F.Cu) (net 27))
 (segment (start 133.35 78.74) (end 133.35 68.58) (width 0.25) (layer F.Cu) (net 27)))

